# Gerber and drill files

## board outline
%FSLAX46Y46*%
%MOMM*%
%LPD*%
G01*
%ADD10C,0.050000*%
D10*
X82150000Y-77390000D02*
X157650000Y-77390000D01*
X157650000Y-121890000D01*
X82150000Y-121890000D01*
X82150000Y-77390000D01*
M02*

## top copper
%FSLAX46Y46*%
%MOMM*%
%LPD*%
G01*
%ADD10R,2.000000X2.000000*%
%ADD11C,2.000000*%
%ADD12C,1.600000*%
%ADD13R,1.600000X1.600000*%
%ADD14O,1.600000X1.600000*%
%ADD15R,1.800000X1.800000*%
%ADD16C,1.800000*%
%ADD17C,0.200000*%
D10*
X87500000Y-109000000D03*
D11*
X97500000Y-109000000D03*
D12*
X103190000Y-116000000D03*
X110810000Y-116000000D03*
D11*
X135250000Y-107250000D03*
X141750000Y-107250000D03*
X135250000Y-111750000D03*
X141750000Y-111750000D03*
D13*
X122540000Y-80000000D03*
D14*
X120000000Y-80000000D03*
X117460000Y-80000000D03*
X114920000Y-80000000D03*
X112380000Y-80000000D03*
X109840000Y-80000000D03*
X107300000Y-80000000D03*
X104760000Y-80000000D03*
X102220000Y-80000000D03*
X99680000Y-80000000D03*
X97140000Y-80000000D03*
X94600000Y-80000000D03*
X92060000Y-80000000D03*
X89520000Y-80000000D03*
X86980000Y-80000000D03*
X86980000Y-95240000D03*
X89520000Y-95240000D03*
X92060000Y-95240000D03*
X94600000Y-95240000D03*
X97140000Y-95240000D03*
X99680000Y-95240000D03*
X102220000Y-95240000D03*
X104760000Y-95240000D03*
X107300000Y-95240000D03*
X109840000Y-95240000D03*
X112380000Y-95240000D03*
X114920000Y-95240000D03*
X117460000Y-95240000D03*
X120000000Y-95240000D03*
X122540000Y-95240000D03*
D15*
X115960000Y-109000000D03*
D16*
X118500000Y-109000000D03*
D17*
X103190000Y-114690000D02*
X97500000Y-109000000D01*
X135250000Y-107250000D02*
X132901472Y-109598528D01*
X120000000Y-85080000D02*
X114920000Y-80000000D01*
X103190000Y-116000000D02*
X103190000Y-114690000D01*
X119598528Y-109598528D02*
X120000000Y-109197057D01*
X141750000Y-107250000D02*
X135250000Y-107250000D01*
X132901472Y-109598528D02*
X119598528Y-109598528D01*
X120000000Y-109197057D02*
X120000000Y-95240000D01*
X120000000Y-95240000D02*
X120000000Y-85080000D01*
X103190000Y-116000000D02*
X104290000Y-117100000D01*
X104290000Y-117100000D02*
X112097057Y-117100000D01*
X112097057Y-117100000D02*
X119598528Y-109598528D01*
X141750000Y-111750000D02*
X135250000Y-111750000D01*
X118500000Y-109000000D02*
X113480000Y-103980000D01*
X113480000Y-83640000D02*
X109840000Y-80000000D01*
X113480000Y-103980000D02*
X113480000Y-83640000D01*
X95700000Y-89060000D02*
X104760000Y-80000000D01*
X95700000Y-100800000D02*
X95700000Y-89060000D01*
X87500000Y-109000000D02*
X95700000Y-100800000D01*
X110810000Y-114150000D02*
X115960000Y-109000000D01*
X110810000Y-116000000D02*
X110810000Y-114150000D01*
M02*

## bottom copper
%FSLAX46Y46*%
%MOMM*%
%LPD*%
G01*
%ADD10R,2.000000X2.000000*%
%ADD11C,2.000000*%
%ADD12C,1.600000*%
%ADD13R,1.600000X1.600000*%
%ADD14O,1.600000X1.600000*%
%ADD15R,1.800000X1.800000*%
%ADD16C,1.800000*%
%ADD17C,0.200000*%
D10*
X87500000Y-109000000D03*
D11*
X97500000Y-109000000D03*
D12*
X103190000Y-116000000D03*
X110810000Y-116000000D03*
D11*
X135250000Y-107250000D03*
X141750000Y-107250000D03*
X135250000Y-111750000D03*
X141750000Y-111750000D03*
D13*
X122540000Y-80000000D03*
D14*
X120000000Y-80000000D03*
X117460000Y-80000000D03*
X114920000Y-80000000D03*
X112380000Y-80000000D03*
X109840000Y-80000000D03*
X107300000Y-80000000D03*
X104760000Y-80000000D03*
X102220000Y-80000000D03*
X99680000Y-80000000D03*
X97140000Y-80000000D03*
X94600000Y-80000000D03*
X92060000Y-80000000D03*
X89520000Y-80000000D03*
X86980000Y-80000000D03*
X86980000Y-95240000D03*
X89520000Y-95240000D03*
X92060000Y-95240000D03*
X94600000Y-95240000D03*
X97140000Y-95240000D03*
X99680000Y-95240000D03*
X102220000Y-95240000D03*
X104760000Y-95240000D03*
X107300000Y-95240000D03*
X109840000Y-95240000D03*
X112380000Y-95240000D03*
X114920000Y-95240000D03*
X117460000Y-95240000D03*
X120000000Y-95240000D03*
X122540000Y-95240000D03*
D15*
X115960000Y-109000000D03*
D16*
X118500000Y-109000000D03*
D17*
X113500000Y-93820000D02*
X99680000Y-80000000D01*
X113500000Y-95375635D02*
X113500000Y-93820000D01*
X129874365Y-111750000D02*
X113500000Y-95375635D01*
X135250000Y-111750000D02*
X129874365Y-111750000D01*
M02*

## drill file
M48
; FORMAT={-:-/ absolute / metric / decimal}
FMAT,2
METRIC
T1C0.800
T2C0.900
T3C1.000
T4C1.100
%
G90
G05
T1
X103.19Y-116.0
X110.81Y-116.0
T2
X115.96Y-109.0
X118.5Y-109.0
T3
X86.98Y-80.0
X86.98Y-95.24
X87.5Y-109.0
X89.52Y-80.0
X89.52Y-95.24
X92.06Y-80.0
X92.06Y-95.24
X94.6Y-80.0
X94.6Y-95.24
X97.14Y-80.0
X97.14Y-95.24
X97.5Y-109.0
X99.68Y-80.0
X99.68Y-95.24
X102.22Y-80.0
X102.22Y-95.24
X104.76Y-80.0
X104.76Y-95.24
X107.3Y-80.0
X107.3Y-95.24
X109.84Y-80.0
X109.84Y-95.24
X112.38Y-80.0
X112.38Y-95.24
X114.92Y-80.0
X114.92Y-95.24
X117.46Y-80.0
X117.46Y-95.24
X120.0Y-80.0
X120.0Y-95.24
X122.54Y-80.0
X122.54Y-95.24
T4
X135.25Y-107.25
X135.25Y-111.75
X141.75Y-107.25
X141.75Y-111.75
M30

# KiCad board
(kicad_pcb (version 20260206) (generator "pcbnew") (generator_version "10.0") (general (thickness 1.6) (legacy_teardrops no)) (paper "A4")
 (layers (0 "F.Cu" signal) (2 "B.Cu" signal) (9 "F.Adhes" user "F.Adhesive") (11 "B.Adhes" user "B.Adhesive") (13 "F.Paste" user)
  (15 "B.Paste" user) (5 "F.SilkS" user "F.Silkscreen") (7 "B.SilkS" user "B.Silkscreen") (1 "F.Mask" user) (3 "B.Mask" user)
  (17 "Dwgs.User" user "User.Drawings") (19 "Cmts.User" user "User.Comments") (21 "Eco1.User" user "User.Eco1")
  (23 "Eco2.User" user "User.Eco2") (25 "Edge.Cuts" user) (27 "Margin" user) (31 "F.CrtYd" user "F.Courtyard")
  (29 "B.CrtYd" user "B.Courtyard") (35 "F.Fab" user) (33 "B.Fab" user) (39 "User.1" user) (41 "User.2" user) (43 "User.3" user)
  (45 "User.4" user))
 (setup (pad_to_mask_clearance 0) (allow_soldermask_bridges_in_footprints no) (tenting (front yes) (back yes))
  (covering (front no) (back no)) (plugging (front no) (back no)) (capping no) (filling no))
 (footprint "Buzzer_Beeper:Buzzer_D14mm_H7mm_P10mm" (layer "F.Cu") (at 87.5 109)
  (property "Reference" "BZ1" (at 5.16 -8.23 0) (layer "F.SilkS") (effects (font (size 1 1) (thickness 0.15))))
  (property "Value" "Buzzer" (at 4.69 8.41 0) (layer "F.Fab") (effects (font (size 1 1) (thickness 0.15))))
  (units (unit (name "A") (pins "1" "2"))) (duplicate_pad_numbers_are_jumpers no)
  (pad "1" thru_hole rect (at 0 0) (size 2 2) (drill 1) (layers "*.Cu" "*.Mask") (remove_unused_layers no) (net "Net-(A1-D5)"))
  (pad "2" thru_hole circle (at 10 0) (size 2 2) (drill 1) (layers "*.Cu" "*.Mask") (remove_unused_layers no) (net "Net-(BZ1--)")))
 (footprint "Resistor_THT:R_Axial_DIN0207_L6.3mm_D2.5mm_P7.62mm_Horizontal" (layer "F.Cu") (at 103.19 116)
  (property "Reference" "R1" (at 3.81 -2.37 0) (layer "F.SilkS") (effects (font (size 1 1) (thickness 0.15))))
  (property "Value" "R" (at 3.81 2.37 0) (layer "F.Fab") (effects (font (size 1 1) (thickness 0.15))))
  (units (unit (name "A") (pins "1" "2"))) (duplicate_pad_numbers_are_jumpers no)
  (pad "1" thru_hole circle (at 0 0) (size 1.6 1.6) (drill 0.8) (layers "*.Cu" "*.Mask") (remove_unused_layers no) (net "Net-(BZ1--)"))
  (pad "2" thru_hole circle (at 7.62 0) (size 1.6 1.6) (drill 0.8) (layers "*.Cu" "*.Mask") (remove_unused_layers no) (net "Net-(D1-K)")))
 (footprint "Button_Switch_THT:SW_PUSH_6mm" (layer "F.Cu") (at 135.25 107.25)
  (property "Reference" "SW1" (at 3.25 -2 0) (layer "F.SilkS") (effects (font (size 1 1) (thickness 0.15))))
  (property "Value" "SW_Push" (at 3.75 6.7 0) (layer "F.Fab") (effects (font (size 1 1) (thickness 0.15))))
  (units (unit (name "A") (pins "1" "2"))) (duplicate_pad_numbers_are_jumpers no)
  (pad "1" thru_hole circle (at 0 0 90) (size 2 2) (drill 1.1) (layers "*.Cu" "*.Mask") (remove_unused_layers no) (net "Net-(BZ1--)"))
  (pad "1" thru_hole circle (at 6.5 0 90) (size 2 2) (drill 1.1) (layers "*.Cu" "*.Mask") (remove_unused_layers no) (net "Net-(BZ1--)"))
  (pad "2" thru_hole circle (at 0 4.5 90) (size 2 2) (drill 1.1) (layers "*.Cu" "*.Mask") (remove_unused_layers no) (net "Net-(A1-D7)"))
  (pad "2" thru_hole circle (at 6.5 4.5 90) (size 2 2) (drill 1.1) (layers "*.Cu" "*.Mask") (remove_unused_layers no) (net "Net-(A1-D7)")))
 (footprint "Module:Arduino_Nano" (layer "F.Cu") (at 122.54 80 -90)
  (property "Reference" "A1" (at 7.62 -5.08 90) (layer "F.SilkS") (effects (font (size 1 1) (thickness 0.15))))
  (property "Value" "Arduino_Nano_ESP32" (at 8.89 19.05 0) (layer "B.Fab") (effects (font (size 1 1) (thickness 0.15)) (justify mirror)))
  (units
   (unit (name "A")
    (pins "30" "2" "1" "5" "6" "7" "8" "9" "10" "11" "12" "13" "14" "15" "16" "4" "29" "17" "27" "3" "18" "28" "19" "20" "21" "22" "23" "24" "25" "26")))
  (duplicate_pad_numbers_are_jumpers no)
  (pad "1" thru_hole rect (at 0 0 270) (size 1.6 1.6) (drill 1) (layers "*.Cu" "*.Mask") (remove_unused_layers no)
   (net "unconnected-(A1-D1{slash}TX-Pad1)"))
  (pad "2" thru_hole oval (at 0 2.54 270) (size 1.6 1.6) (drill 1) (layers "*.Cu" "*.Mask") (remove_unused_layers no)
   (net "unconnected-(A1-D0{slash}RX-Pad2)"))
  (pad "3" thru_hole oval (at 0 5.08 270) (size 1.6 1.6) (drill 1) (layers "*.Cu" "*.Mask") (remove_unused_layers no)
   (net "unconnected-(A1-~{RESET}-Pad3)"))
  (pad "4" thru_hole oval (at 0 7.62 270) (size 1.6 1.6) (drill 1) (layers "*.Cu" "*.Mask") (remove_unused_layers no) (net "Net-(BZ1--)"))
  (pad "5" thru_hole oval (at 0 10.16 270) (size 1.6 1.6) (drill 1) (layers "*.Cu" "*.Mask") (remove_unused_layers no)
   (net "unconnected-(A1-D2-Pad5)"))
  (pad "6" thru_hole oval (at 0 12.7 270) (size 1.6 1.6) (drill 1) (layers "*.Cu" "*.Mask") (remove_unused_layers no) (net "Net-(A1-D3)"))
  (pad "7" thru_hole oval (at 0 15.24 270) (size 1.6 1.6) (drill 1) (layers "*.Cu" "*.Mask") (remove_unused_layers no)
   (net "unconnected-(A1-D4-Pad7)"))
  (pad "8" thru_hole oval (at 0 17.78 270) (size 1.6 1.6) (drill 1) (layers "*.Cu" "*.Mask") (remove_unused_layers no) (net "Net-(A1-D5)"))
  (pad "9" thru_hole oval (at 0 20.32 270) (size 1.6 1.6) (drill 1) (layers "*.Cu" "*.Mask") (remove_unused_layers no)
   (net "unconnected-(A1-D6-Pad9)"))
  (pad "10" thru_hole oval (at 0 22.86 270) (size 1.6 1.6) (drill 1) (layers "*.Cu" "*.Mask") (remove_unused_layers no) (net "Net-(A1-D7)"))
  (pad "11" thru_hole oval (at 0 25.4 270) (size 1.6 1.6) (drill 1) (layers "*.Cu" "*.Mask") (remove_unused_layers no)
   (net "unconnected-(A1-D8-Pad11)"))
  (pad "12" thru_hole oval (at 0 27.94 270) (size 1.6 1.6) (drill 1) (layers "*.Cu" "*.Mask") (remove_unused_layers no)
   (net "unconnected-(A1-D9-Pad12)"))
  (pad "13" thru_hole oval (at 0 30.48 270) (size 1.6 1.6) (drill 1) (layers "*.Cu" "*.Mask") (remove_unused_layers no)
   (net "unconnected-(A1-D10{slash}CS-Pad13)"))
  (pad "14" thru_hole oval (at 0 33.02 270) (size 1.6 1.6) (drill 1) (layers "*.Cu" "*.Mask") (remove_unused_layers no)
   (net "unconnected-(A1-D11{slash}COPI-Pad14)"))
  (pad "15" thru_hole oval (at 0 35.56 270) (size 1.6 1.6) (drill 1) (layers "*.Cu" "*.Mask") (remove_unused_layers no)
   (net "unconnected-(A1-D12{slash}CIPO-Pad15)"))
  (pad "16" thru_hole oval (at 15.24 35.56 270) (size 1.6 1.6) (drill 1) (layers "*.Cu" "*.Mask") (remove_unused_layers no)
   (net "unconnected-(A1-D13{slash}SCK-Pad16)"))
  (pad "17" thru_hole oval (at 15.24 33.02 270) (size 1.6 1.6) (drill 1) (layers "*.Cu" "*.Mask") (remove_unused_layers no)
   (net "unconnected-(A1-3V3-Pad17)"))
  (pad "18" thru_hole oval (at 15.24 30.48 270) (size 1.6 1.6) (drill 1) (layers "*.Cu" "*.Mask") (remove_unused_layers no)
   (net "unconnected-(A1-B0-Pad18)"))
  (pad "19" thru_hole oval (at 15.24 27.94 270) (size 1.6 1.6) (drill 1) (layers "*.Cu" "*.Mask") (remove_unused_layers no)
   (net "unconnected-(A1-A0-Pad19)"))
  (pad "20" thru_hole oval (at 15.24 25.4 270) (size 1.6 1.6) (drill 1) (layers "*.Cu" "*.Mask") (remove_unused_layers no)
   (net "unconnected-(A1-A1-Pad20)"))
  (pad "21" thru_hole oval (at 15.24 22.86 270) (size 1.6 1.6) (drill 1) (layers "*.Cu" "*.Mask") (remove_unused_layers no)
   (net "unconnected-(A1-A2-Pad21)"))
  (pad "22" thru_hole oval (at 15.24 20.32 270) (size 1.6 1.6) (drill 1) (layers "*.Cu" "*.Mask") (remove_unused_layers no)
   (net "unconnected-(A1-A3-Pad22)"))
  (pad "23" thru_hole oval (at 15.24 17.78 270) (size 1.6 1.6) (drill 1) (layers "*.Cu" "*.Mask") (remove_unused_layers no)
   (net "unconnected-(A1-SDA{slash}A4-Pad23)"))
  (pad "24" thru_hole oval (at 15.24 15.24 270) (size 1.6 1.6) (drill 1) (layers "*.Cu" "*.Mask") (remove_unused_layers no)
   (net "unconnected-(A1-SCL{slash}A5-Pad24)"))
  (pad "25" thru_hole oval (at 15.24 12.7 270) (size 1.6 1.6) (drill 1) (layers "*.Cu" "*.Mask") (remove_unused_layers no)
   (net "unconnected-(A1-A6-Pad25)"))
  (pad "26" thru_hole oval (at 15.24 10.16 270) (size 1.6 1.6) (drill 1) (layers "*.Cu" "*.Mask") (remove_unused_layers no)
   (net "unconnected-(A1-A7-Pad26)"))
  (pad "27" thru_hole oval (at 15.24 7.62 270) (size 1.6 1.6) (drill 1) (layers "*.Cu" "*.Mask") (remove_unused_layers no)
   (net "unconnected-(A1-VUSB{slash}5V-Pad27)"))
  (pad "28" thru_hole oval (at 15.24 5.08 270) (size 1.6 1.6) (drill 1) (layers "*.Cu" "*.Mask") (remove_unused_layers no)
   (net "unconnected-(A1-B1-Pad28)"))
  (pad "29" thru_hole oval (at 15.24 2.54 270) (size 1.6 1.6) (drill 1) (layers "*.Cu" "*.Mask") (remove_unused_layers no)
   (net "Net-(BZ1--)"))
  (pad "30" thru_hole oval (at 15.24 0 270) (size 1.6 1.6) (drill 1) (layers "*.Cu" "*.Mask") (remove_unused_layers no)
   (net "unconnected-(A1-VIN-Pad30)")))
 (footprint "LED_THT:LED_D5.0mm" (layer "F.Cu") (at 115.96 109)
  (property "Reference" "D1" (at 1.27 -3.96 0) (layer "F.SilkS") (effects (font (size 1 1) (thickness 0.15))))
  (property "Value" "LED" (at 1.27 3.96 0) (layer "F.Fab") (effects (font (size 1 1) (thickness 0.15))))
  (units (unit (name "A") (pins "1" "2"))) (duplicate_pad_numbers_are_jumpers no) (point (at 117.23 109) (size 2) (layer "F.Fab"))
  (pad "1" thru_hole rect (at 0 0) (size 1.8 1.8) (drill 0.9) (layers "*.Cu" "*.Mask") (remove_unused_layers no) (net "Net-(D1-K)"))
  (pad "2" thru_hole circle (at 2.54 0) (size 1.8 1.8) (drill 0.9) (layers "*.Cu" "*.Mask") (remove_unused_layers no) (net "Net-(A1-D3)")))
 (gr_rect (start 82.15 77.39) (end 157.65 121.89) (stroke (width 0.05) (type default)) (fill no) (layer "Edge.Cuts"))
 (segment (start 103.19 114.69) (end 97.5 109) (width 0.2) (layer "F.Cu") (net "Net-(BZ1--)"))
 (segment (start 135.25 107.25) (end 132.901472 109.598528) (width 0.2) (layer "F.Cu") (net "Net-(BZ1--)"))
 (segment (start 120 85.08) (end 114.92 80) (width 0.2) (layer "F.Cu") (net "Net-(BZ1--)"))
 (segment (start 103.19 116) (end 103.19 114.69) (width 0.2) (layer "F.Cu") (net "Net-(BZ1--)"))
 (segment (start 119.598528 109.598528) (end 120 109.197057) (width 0.2) (layer "F.Cu") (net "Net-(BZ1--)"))
 (segment (start 141.75 107.25) (end 135.25 107.25) (width 0.2) (layer "F.Cu") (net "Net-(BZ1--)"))
 (segment (start 132.901472 109.598528) (end 119.598528 109.598528) (width 0.2) (layer "F.Cu") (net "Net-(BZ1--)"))
 (segment (start 120 109.197057) (end 120 95.24) (width 0.2) (layer "F.Cu") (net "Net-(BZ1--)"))
 (segment (start 120 95.24) (end 120 85.08) (width 0.2) (layer "F.Cu") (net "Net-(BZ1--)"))
 (segment (start 103.19 116) (end 104.29 117.1) (width 0.2) (layer "F.Cu") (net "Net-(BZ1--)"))
 (segment (start 104.29 117.1) (end 112.097057 117.1) (width 0.2) (layer "F.Cu") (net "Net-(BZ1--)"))
 (segment (start 112.097057 117.1) (end 119.598528 109.598528) (width 0.2) (layer "F.Cu") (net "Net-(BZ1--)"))
 (segment (start 141.75 111.75) (end 135.25 111.75) (width 0.2) (layer "F.Cu") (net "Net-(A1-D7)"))
 (segment (start 113.5 93.82) (end 99.68 80) (width 0.2) (layer "B.Cu") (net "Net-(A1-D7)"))
 (segment (start 113.5 95.375635) (end 113.5 93.82) (width 0.2) (layer "B.Cu") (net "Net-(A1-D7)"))
 (segment (start 129.874365 111.75) (end 113.5 95.375635) (width 0.2) (layer "B.Cu") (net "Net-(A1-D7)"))
 (segment (start 135.25 111.75) (end 129.874365 111.75) (width 0.2) (layer "B.Cu") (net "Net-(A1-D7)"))
 (segment (start 118.5 109) (end 113.48 103.98) (width 0.2) (layer "F.Cu") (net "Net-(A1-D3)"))
 (segment (start 113.48 83.64) (end 109.84 80) (width 0.2) (layer "F.Cu") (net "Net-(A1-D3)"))
 (segment (start 113.48 103.98) (end 113.48 83.64) (width 0.2) (layer "F.Cu") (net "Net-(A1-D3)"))
 (segment (start 95.7 89.06) (end 104.76 80) (width 0.2) (layer "F.Cu") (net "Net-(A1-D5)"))
 (segment (start 95.7 100.8) (end 95.7 89.06) (width 0.2) (layer "F.Cu") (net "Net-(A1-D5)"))
 (segment (start 87.5 109) (end 95.7 100.8) (width 0.2) (layer "F.Cu") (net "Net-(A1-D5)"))
 (segment (start 110.81 114.15) (end 115.96 109) (width 0.2) (layer "F.Cu") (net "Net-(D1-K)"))
 (segment (start 110.81 116) (end 110.81 114.15) (width 0.2) (layer "F.Cu") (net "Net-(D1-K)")))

